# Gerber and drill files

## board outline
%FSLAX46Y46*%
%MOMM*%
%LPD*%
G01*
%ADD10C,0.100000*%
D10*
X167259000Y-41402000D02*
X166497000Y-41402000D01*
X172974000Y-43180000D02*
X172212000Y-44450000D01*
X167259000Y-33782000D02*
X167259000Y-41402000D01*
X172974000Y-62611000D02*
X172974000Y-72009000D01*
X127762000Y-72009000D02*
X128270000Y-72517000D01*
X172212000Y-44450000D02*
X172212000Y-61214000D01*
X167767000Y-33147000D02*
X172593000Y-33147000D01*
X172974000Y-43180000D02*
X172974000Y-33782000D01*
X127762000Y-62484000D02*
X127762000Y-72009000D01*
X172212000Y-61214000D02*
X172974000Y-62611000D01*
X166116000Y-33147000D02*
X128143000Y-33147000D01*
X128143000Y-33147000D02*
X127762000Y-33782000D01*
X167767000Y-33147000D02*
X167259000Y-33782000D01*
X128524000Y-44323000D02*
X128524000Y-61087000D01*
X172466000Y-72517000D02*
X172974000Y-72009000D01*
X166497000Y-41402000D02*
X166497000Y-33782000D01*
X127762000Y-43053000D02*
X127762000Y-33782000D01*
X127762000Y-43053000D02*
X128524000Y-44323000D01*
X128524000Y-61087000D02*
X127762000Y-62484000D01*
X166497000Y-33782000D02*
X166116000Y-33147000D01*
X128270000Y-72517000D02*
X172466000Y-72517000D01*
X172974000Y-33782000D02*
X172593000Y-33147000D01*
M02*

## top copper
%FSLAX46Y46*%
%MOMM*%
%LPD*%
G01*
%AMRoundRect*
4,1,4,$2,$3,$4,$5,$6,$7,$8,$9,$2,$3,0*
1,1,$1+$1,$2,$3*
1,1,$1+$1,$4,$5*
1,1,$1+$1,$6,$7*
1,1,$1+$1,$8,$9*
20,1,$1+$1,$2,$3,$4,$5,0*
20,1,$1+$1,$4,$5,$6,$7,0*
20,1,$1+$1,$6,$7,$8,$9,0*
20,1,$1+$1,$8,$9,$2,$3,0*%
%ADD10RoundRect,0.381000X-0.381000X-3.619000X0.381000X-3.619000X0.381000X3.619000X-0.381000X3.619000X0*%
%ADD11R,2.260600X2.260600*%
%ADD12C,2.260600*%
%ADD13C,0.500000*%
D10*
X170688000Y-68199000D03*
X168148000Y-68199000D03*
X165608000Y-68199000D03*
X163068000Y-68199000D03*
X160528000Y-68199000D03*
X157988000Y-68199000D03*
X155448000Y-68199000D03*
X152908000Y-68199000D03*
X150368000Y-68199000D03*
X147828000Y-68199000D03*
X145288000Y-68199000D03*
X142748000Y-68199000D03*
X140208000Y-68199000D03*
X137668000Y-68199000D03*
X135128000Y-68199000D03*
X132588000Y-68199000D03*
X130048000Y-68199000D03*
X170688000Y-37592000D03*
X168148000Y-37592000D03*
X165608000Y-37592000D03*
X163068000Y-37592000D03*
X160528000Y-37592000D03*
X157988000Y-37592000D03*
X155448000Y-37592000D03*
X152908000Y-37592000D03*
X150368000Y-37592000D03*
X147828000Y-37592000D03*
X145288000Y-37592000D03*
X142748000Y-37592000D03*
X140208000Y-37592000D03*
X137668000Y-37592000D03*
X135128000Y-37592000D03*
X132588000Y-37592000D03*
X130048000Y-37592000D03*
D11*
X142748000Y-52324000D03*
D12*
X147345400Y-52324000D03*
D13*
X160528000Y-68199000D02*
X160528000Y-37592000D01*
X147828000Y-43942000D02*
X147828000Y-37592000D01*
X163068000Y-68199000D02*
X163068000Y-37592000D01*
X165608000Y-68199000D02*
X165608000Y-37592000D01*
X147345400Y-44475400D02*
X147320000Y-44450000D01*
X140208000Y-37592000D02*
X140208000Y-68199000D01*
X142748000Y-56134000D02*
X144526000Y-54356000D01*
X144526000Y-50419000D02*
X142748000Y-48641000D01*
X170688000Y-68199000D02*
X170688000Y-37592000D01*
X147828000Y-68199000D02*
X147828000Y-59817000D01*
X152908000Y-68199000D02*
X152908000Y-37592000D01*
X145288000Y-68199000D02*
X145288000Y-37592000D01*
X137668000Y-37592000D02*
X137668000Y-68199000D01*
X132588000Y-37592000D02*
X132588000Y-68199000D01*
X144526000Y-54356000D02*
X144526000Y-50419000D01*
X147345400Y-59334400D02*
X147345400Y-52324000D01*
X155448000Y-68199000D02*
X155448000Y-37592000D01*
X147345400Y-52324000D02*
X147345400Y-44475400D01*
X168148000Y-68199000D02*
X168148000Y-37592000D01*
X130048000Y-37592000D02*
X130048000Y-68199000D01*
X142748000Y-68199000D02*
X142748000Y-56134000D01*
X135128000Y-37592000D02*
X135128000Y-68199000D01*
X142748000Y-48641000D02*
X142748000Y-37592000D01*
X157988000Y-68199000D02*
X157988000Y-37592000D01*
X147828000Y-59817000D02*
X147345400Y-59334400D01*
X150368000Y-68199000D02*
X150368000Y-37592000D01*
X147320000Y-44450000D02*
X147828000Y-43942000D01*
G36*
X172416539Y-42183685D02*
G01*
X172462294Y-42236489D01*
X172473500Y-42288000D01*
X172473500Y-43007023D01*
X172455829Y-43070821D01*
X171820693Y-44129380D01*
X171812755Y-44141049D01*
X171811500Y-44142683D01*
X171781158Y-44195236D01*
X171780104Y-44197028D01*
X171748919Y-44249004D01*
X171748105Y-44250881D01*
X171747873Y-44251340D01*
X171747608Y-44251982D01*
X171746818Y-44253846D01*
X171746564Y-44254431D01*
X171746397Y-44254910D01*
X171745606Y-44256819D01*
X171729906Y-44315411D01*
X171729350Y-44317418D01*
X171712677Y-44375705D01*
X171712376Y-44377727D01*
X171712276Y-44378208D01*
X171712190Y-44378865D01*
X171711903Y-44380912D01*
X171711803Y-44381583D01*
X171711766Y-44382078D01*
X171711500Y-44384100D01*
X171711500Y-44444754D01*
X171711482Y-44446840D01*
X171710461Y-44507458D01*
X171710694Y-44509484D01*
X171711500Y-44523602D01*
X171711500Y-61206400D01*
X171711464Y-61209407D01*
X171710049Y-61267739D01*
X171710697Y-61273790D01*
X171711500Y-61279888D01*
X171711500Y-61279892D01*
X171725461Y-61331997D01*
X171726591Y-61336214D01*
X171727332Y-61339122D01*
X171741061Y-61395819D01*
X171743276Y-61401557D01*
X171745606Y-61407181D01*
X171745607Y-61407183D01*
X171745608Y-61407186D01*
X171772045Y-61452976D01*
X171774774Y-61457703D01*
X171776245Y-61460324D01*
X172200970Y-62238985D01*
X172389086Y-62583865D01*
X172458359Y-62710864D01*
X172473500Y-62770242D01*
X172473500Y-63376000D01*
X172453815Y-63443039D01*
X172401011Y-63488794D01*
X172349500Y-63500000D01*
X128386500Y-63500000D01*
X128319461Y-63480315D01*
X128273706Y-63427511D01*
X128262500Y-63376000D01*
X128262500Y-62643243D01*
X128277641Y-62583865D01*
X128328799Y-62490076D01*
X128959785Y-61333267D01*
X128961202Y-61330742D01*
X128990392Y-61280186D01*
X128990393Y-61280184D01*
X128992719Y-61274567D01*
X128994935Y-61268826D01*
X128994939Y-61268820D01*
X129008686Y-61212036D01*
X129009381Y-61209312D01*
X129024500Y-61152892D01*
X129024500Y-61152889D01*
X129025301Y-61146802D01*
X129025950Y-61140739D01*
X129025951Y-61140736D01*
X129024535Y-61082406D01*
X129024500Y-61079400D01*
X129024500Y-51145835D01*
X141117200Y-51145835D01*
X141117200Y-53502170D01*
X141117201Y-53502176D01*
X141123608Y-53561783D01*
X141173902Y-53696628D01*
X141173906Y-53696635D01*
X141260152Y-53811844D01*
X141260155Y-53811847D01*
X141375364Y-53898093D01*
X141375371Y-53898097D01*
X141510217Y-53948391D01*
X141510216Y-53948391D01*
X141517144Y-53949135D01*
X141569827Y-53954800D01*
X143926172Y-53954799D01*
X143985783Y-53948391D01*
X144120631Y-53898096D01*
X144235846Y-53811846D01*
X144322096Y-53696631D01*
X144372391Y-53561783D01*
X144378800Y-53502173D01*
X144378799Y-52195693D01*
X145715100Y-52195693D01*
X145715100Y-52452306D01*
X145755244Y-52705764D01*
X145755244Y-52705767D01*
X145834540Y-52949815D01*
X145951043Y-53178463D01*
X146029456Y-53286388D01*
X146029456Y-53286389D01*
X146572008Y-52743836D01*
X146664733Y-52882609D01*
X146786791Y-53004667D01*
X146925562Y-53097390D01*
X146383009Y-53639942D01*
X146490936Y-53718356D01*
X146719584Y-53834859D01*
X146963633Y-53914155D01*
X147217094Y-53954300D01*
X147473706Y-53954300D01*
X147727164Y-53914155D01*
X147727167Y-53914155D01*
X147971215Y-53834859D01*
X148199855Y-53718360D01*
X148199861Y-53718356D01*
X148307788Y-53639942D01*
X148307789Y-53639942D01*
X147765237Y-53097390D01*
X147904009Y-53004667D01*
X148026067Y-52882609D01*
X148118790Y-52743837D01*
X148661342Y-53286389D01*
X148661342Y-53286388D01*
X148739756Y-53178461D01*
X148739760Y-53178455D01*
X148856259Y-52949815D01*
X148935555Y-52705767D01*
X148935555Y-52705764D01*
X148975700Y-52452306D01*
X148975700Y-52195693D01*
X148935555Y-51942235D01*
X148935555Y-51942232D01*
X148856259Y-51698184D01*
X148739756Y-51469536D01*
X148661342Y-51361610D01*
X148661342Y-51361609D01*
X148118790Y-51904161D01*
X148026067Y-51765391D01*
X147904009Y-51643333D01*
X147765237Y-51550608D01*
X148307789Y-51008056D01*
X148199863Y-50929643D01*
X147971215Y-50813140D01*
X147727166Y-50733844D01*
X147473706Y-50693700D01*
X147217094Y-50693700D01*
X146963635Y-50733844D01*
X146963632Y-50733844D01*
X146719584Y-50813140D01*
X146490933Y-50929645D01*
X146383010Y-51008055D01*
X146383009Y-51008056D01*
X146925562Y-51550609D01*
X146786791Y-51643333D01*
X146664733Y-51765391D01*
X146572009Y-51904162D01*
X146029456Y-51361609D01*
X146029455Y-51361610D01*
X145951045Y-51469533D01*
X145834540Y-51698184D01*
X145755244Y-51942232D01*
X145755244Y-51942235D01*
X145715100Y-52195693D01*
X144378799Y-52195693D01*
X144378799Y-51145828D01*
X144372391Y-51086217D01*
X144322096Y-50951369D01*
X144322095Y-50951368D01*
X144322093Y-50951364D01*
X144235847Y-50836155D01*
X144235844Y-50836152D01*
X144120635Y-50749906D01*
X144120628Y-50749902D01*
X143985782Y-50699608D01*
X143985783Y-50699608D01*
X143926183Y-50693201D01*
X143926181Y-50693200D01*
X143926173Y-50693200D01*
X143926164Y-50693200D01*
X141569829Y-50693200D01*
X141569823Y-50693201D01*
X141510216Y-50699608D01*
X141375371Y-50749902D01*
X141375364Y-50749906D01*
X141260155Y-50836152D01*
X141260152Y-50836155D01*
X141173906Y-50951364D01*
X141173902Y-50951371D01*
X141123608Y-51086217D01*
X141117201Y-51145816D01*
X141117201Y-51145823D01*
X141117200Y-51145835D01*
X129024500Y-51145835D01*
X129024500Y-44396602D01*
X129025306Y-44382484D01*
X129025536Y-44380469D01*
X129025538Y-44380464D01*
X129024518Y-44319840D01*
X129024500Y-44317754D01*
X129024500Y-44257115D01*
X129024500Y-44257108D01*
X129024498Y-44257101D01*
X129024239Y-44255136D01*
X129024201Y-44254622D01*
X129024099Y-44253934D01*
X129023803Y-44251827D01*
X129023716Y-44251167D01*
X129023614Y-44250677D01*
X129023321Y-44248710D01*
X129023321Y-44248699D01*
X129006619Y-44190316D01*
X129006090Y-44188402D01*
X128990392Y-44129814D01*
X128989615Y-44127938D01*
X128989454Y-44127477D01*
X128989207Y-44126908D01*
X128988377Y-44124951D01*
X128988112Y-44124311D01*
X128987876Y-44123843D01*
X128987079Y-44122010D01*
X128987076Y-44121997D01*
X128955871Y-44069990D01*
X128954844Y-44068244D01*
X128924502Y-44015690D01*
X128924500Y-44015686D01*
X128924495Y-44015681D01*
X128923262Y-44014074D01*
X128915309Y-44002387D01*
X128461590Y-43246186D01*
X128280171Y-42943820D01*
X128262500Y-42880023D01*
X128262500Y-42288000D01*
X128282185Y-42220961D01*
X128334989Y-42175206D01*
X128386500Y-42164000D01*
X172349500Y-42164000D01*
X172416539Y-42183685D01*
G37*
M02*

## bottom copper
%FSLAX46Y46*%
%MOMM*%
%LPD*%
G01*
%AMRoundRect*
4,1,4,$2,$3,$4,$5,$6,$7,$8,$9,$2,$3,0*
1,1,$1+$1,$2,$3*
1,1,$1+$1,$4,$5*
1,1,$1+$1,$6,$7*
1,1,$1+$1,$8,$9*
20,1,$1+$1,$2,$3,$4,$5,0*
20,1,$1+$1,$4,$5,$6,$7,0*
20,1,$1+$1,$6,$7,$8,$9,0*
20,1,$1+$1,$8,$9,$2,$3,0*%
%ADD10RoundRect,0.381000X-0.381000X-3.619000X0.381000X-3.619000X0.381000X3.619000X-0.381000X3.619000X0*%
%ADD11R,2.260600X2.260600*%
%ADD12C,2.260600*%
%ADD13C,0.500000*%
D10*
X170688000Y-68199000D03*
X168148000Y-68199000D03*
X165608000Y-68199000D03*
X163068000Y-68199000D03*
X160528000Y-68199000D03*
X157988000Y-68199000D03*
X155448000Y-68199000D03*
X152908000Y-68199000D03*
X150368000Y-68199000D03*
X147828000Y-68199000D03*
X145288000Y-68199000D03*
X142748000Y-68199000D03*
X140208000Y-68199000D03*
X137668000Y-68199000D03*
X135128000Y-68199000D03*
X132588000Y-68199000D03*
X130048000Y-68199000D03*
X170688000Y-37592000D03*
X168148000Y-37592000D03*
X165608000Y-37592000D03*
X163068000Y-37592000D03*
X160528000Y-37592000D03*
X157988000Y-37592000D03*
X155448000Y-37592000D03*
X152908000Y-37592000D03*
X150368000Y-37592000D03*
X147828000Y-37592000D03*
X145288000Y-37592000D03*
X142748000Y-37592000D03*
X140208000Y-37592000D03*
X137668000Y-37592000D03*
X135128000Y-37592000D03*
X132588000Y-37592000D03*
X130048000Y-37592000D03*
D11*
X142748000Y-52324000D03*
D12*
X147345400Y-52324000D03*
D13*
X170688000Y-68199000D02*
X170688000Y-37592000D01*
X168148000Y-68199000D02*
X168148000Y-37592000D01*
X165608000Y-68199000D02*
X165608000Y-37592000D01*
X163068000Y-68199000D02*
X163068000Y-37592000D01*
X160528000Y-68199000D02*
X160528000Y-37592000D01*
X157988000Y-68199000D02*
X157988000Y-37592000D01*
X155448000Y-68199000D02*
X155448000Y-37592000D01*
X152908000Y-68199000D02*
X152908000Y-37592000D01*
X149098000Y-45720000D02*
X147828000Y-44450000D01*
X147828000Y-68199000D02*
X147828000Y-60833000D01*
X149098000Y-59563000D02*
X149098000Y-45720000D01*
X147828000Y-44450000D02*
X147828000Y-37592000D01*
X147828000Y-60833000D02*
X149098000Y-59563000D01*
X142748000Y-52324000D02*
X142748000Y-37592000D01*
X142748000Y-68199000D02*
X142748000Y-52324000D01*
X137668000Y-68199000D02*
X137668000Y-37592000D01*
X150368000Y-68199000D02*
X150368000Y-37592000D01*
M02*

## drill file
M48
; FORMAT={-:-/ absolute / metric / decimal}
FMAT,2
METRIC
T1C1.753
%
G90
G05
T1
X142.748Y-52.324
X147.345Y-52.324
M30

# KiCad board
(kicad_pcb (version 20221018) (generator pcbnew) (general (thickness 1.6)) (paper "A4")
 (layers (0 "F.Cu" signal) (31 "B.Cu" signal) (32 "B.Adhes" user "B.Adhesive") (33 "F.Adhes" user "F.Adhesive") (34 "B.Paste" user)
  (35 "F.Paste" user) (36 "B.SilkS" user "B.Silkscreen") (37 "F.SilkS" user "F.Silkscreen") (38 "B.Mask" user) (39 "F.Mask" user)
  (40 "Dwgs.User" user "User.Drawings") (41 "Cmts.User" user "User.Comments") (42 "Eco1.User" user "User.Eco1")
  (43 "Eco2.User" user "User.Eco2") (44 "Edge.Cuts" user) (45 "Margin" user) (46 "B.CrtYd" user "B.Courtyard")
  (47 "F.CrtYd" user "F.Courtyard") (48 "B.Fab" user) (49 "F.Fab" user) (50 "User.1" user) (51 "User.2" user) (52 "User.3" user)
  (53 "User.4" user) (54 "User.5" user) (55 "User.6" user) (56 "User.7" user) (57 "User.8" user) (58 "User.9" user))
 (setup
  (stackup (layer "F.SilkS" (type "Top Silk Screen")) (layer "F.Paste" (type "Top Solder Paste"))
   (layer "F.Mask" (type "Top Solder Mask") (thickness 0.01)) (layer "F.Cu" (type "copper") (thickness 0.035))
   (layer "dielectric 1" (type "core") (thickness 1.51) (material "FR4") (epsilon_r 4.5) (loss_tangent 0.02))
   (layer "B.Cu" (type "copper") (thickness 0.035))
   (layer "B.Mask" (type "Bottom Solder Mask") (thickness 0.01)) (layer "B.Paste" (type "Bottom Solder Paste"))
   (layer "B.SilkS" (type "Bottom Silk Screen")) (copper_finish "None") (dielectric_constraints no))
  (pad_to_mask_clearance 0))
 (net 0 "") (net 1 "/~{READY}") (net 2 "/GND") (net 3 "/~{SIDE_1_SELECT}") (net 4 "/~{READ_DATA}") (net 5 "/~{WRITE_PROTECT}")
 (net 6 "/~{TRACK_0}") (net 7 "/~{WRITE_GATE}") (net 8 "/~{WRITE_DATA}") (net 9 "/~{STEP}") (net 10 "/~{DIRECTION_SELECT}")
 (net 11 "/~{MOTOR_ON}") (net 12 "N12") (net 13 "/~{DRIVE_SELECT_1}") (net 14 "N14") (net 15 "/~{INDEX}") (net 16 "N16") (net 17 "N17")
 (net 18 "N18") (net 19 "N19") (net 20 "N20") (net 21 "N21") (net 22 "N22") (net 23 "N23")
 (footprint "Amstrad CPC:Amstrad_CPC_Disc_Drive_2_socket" (layer "F.Cu") (at 157.988 74.803)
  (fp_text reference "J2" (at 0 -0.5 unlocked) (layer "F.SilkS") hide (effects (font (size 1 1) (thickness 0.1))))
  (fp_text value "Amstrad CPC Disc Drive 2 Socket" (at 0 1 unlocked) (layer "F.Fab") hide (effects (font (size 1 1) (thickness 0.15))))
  (pad "1" smd roundrect (at 12.7 -6.604) (size 1.524 8) (layers "B.Cu" "B.Paste" "B.Mask") (roundrect_rratio 0.25) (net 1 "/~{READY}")
   (thermal_bridge_angle 45))
  (pad "2" smd roundrect (at 12.7 -6.604) (size 1.524 8) (layers "F.Cu" "F.Paste" "F.Mask") (roundrect_rratio 0.25) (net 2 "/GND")
   (thermal_bridge_angle 45))
  (pad "3" smd roundrect (at 10.16 -6.604) (size 1.524 8) (layers "B.Cu" "B.Paste" "B.Mask") (roundrect_rratio 0.25)
   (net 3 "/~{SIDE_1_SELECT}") (thermal_bridge_angle 45))
  (pad "4" smd roundrect (at 10.16 -6.604) (size 1.524 8) (layers "F.Cu" "F.Paste" "F.Mask") (roundrect_rratio 0.25) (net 2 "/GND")
   (thermal_bridge_angle 45))
  (pad "5" smd roundrect (at 7.62 -6.604) (size 1.524 8) (layers "B.Cu" "B.Paste" "B.Mask") (roundrect_rratio 0.25) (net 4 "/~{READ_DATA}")
   (thermal_bridge_angle 45))
  (pad "6" smd roundrect (at 7.62 -6.604) (size 1.524 8) (layers "F.Cu" "F.Paste" "F.Mask") (roundrect_rratio 0.25) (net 2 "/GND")
   (thermal_bridge_angle 45))
  (pad "7" smd roundrect (at 5.08 -6.604) (size 1.524 8) (layers "B.Cu" "B.Paste" "B.Mask") (roundrect_rratio 0.25)
   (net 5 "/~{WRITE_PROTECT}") (thermal_bridge_angle 45))
  (pad "8" smd roundrect (at 5.08 -6.604) (size 1.524 8) (layers "F.Cu" "F.Paste" "F.Mask") (roundrect_rratio 0.25) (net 2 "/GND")
   (thermal_bridge_angle 45))
  (pad "9" smd roundrect (at 2.54 -6.604) (size 1.524 8) (layers "B.Cu" "B.Paste" "B.Mask") (roundrect_rratio 0.25) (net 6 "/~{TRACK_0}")
   (thermal_bridge_angle 45))
  (pad "10" smd roundrect (at 2.54 -6.604) (size 1.524 8) (layers "F.Cu" "F.Paste" "F.Mask") (roundrect_rratio 0.25) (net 2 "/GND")
   (thermal_bridge_angle 45))
  (pad "11" smd roundrect (at 0 -6.604) (size 1.524 8) (layers "B.Cu" "B.Paste" "B.Mask") (roundrect_rratio 0.25) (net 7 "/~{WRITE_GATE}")
   (thermal_bridge_angle 45))
  (pad "12" smd roundrect (at 0 -6.604) (size 1.524 8) (layers "F.Cu" "F.Paste" "F.Mask") (roundrect_rratio 0.25) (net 2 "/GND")
   (thermal_bridge_angle 45))
  (pad "13" smd roundrect (at -2.54 -6.604) (size 1.524 8) (layers "B.Cu" "B.Paste" "B.Mask") (roundrect_rratio 0.25)
   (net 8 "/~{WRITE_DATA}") (thermal_bridge_angle 45))
  (pad "14" smd roundrect (at -2.54 -6.604) (size 1.524 8) (layers "F.Cu" "F.Paste" "F.Mask") (roundrect_rratio 0.25) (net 2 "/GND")
   (thermal_bridge_angle 45))
  (pad "15" smd roundrect (at -5.08 -6.604) (size 1.524 8) (layers "B.Cu" "B.Paste" "B.Mask") (roundrect_rratio 0.25) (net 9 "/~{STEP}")
   (thermal_bridge_angle 45))
  (pad "16" smd roundrect (at -5.08 -6.604) (size 1.524 8) (layers "F.Cu" "F.Paste" "F.Mask") (roundrect_rratio 0.25) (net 2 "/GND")
   (thermal_bridge_angle 45))
  (pad "17" smd roundrect (at -7.62 -6.604) (size 1.524 8) (layers "B.Cu" "B.Paste" "B.Mask") (roundrect_rratio 0.25)
   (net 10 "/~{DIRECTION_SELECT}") (thermal_bridge_angle 45))
  (pad "18" smd roundrect (at -7.62 -6.604) (size 1.524 8) (layers "F.Cu" "F.Paste" "F.Mask") (roundrect_rratio 0.25) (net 2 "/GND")
   (thermal_bridge_angle 45))
  (pad "19" smd roundrect (at -10.16 -6.604) (size 1.524 8) (layers "B.Cu" "B.Paste" "B.Mask") (roundrect_rratio 0.25)
   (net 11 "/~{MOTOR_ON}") (thermal_bridge_angle 45))
  (pad "20" smd roundrect (at -10.16 -6.604) (size 1.524 8) (layers "F.Cu" "F.Paste" "F.Mask") (roundrect_rratio 0.25) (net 2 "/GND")
   (thermal_bridge_angle 45))
  (pad "21" smd roundrect (at -12.7 -6.604) (size 1.524 8) (layers "B.Cu" "B.Paste" "B.Mask") (roundrect_rratio 0.25) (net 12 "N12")
   (thermal_bridge_angle 45))
  (pad "22" smd roundrect (at -12.7 -6.604) (size 1.524 8) (layers "F.Cu" "F.Paste" "F.Mask") (roundrect_rratio 0.25) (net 2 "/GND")
   (thermal_bridge_angle 45))
  (pad "23" smd roundrect (at -15.24 -6.604) (size 1.524 8) (layers "B.Cu" "B.Paste" "B.Mask") (roundrect_rratio 0.25)
   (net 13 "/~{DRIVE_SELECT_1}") (thermal_bridge_angle 45))
  (pad "24" smd roundrect (at -15.24 -6.604) (size 1.524 8) (layers "F.Cu" "F.Paste" "F.Mask") (roundrect_rratio 0.25) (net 2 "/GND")
   (thermal_bridge_angle 45))
  (pad "25" smd roundrect (at -17.78 -6.604) (size 1.524 8) (layers "B.Cu" "B.Paste" "B.Mask") (roundrect_rratio 0.25) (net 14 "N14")
   (thermal_bridge_angle 45))
  (pad "26" smd roundrect (at -17.78 -6.604) (size 1.524 8) (layers "F.Cu" "F.Paste" "F.Mask") (roundrect_rratio 0.25) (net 2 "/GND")
   (thermal_bridge_angle 45))
  (pad "27" smd roundrect (at -20.32 -6.604) (size 1.524 8) (layers "B.Cu" "B.Paste" "B.Mask") (roundrect_rratio 0.25) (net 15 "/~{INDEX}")
   (thermal_bridge_angle 45))
  (pad "28" smd roundrect (at -20.32 -6.604) (size 1.524 8) (layers "F.Cu" "F.Paste" "F.Mask") (roundrect_rratio 0.25) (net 2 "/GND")
   (thermal_bridge_angle 45))
  (pad "29" smd roundrect (at -22.86 -6.604) (size 1.524 8) (layers "B.Cu" "B.Paste" "B.Mask") (roundrect_rratio 0.25) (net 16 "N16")
   (thermal_bridge_angle 45))
  (pad "30" smd roundrect (at -22.86 -6.604) (size 1.524 8) (layers "F.Cu" "F.Paste" "F.Mask") (roundrect_rratio 0.25) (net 2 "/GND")
   (thermal_bridge_angle 45))
  (pad "31" smd roundrect (at -25.4 -6.604) (size 1.524 8) (layers "B.Cu" "B.Paste" "B.Mask") (roundrect_rratio 0.25) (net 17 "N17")
   (thermal_bridge_angle 45))
  (pad "32" smd roundrect (at -25.4 -6.604) (size 1.524 8) (layers "F.Cu" "F.Paste" "F.Mask") (roundrect_rratio 0.25) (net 2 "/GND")
   (thermal_bridge_angle 45))
  (pad "33" smd roundrect (at -27.94 -6.604) (size 1.524 8) (layers "B.Cu" "B.Paste" "B.Mask") (roundrect_rratio 0.25) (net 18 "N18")
   (thermal_bridge_angle 45))
  (pad "34" smd roundrect (at -27.94 -6.604) (size 1.524 8) (layers "F.Cu" "F.Paste" "F.Mask") (roundrect_rratio 0.25) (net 2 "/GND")
   (thermal_bridge_angle 45)))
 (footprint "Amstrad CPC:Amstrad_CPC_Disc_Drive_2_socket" (layer "F.Cu") (at 157.988 44.196)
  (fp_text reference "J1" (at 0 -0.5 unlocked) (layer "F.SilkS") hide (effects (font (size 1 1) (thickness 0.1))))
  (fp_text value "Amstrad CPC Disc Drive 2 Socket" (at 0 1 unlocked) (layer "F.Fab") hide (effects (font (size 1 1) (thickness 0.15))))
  (pad "1" smd roundrect (at 12.7 -6.604) (size 1.524 8) (layers "B.Cu" "B.Paste" "B.Mask") (roundrect_rratio 0.25) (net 1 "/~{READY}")
   (thermal_bridge_angle 45))
  (pad "2" smd roundrect (at 12.7 -6.604) (size 1.524 8) (layers "F.Cu" "F.Paste" "F.Mask") (roundrect_rratio 0.25) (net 2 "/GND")
   (thermal_bridge_angle 45))
  (pad "3" smd roundrect (at 10.16 -6.604) (size 1.524 8) (layers "B.Cu" "B.Paste" "B.Mask") (roundrect_rratio 0.25)
   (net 3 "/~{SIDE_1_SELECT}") (thermal_bridge_angle 45))
  (pad "4" smd roundrect (at 10.16 -6.604) (size 1.524 8) (layers "F.Cu" "F.Paste" "F.Mask") (roundrect_rratio 0.25) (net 2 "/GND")
   (thermal_bridge_angle 45))
  (pad "5" smd roundrect (at 7.62 -6.604) (size 1.524 8) (layers "B.Cu" "B.Paste" "B.Mask") (roundrect_rratio 0.25) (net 4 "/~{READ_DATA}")
   (thermal_bridge_angle 45))
  (pad "6" smd roundrect (at 7.62 -6.604) (size 1.524 8) (layers "F.Cu" "F.Paste" "F.Mask") (roundrect_rratio 0.25) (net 2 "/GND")
   (thermal_bridge_angle 45))
  (pad "7" smd roundrect (at 5.08 -6.604) (size 1.524 8) (layers "B.Cu" "B.Paste" "B.Mask") (roundrect_rratio 0.25)
   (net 5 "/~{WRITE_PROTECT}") (thermal_bridge_angle 45))
  (pad "8" smd roundrect (at 5.08 -6.604) (size 1.524 8) (layers "F.Cu" "F.Paste" "F.Mask") (roundrect_rratio 0.25) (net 2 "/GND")
   (thermal_bridge_angle 45))
  (pad "9" smd roundrect (at 2.54 -6.604) (size 1.524 8) (layers "B.Cu" "B.Paste" "B.Mask") (roundrect_rratio 0.25) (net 6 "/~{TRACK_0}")
   (thermal_bridge_angle 45))
  (pad "10" smd roundrect (at 2.54 -6.604) (size 1.524 8) (layers "F.Cu" "F.Paste" "F.Mask") (roundrect_rratio 0.25) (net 2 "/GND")
   (thermal_bridge_angle 45))
  (pad "11" smd roundrect (at 0 -6.604) (size 1.524 8) (layers "B.Cu" "B.Paste" "B.Mask") (roundrect_rratio 0.25) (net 7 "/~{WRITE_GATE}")
   (thermal_bridge_angle 45))
  (pad "12" smd roundrect (at 0 -6.604) (size 1.524 8) (layers "F.Cu" "F.Paste" "F.Mask") (roundrect_rratio 0.25) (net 2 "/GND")
   (thermal_bridge_angle 45))
  (pad "13" smd roundrect (at -2.54 -6.604) (size 1.524 8) (layers "B.Cu" "B.Paste" "B.Mask") (roundrect_rratio 0.25)
   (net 8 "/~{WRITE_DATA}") (thermal_bridge_angle 45))
  (pad "14" smd roundrect (at -2.54 -6.604) (size 1.524 8) (layers "F.Cu" "F.Paste" "F.Mask") (roundrect_rratio 0.25) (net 2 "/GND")
   (thermal_bridge_angle 45))
  (pad "15" smd roundrect (at -5.08 -6.604) (size 1.524 8) (layers "B.Cu" "B.Paste" "B.Mask") (roundrect_rratio 0.25) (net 9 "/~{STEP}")
   (thermal_bridge_angle 45))
  (pad "16" smd roundrect (at -5.08 -6.604) (size 1.524 8) (layers "F.Cu" "F.Paste" "F.Mask") (roundrect_rratio 0.25) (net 2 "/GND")
   (thermal_bridge_angle 45))
  (pad "17" smd roundrect (at -7.62 -6.604) (size 1.524 8) (layers "B.Cu" "B.Paste" "B.Mask") (roundrect_rratio 0.25)
   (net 10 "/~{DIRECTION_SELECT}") (thermal_bridge_angle 45))
  (pad "18" smd roundrect (at -7.62 -6.604) (size 1.524 8) (layers "F.Cu" "F.Paste" "F.Mask") (roundrect_rratio 0.25) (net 2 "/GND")
   (thermal_bridge_angle 45))
  (pad "19" smd roundrect (at -10.16 -6.604) (size 1.524 8) (layers "B.Cu" "B.Paste" "B.Mask") (roundrect_rratio 0.25)
   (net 11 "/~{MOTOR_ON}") (thermal_bridge_angle 45))
  (pad "20" smd roundrect (at -10.16 -6.604) (size 1.524 8) (layers "F.Cu" "F.Paste" "F.Mask") (roundrect_rratio 0.25) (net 2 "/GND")
   (thermal_bridge_angle 45))
  (pad "21" smd roundrect (at -12.7 -6.604) (size 1.524 8) (layers "B.Cu" "B.Paste" "B.Mask") (roundrect_rratio 0.25) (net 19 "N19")
   (thermal_bridge_angle 45))
  (pad "22" smd roundrect (at -12.7 -6.604) (size 1.524 8) (layers "F.Cu" "F.Paste" "F.Mask") (roundrect_rratio 0.25) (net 2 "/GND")
   (thermal_bridge_angle 45))
  (pad "23" smd roundrect (at -15.24 -6.604) (size 1.524 8) (layers "B.Cu" "B.Paste" "B.Mask") (roundrect_rratio 0.25)
   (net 13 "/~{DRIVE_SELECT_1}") (thermal_bridge_angle 45))
  (pad "24" smd roundrect (at -15.24 -6.604) (size 1.524 8) (layers "F.Cu" "F.Paste" "F.Mask") (roundrect_rratio 0.25) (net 2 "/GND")
   (thermal_bridge_angle 45))
  (pad "25" smd roundrect (at -17.78 -6.604) (size 1.524 8) (layers "B.Cu" "B.Paste" "B.Mask") (roundrect_rratio 0.25) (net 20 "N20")
   (thermal_bridge_angle 45))
  (pad "26" smd roundrect (at -17.78 -6.604) (size 1.524 8) (layers "F.Cu" "F.Paste" "F.Mask") (roundrect_rratio 0.25) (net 2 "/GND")
   (thermal_bridge_angle 45))
  (pad "27" smd roundrect (at -20.32 -6.604) (size 1.524 8) (layers "B.Cu" "B.Paste" "B.Mask") (roundrect_rratio 0.25) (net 15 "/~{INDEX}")
   (thermal_bridge_angle 45))
  (pad "28" smd roundrect (at -20.32 -6.604) (size 1.524 8) (layers "F.Cu" "F.Paste" "F.Mask") (roundrect_rratio 0.25) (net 2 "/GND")
   (thermal_bridge_angle 45))
  (pad "29" smd roundrect (at -22.86 -6.604) (size 1.524 8) (layers "B.Cu" "B.Paste" "B.Mask") (roundrect_rratio 0.25) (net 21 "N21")
   (thermal_bridge_angle 45))
  (pad "30" smd roundrect (at -22.86 -6.604) (size 1.524 8) (layers "F.Cu" "F.Paste" "F.Mask") (roundrect_rratio 0.25) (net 2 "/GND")
   (thermal_bridge_angle 45))
  (pad "31" smd roundrect (at -25.4 -6.604) (size 1.524 8) (layers "B.Cu" "B.Paste" "B.Mask") (roundrect_rratio 0.25) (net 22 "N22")
   (thermal_bridge_angle 45))
  (pad "32" smd roundrect (at -25.4 -6.604) (size 1.524 8) (layers "F.Cu" "F.Paste" "F.Mask") (roundrect_rratio 0.25) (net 2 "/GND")
   (thermal_bridge_angle 45))
  (pad "33" smd roundrect (at -27.94 -6.604) (size 1.524 8) (layers "B.Cu" "B.Paste" "B.Mask") (roundrect_rratio 0.25) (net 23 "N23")
   (thermal_bridge_angle 45))
  (pad "34" smd roundrect (at -27.94 -6.604) (size 1.524 8) (layers "F.Cu" "F.Paste" "F.Mask") (roundrect_rratio 0.25) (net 2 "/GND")
   (thermal_bridge_angle 45)))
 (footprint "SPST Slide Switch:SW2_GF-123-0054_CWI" (layer "F.Cu") (at 142.748 52.324 90)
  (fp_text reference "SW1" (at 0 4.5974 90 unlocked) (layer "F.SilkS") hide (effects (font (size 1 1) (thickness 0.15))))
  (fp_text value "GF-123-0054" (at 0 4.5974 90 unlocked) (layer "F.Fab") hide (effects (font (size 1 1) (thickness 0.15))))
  (pad "1" thru_hole rect (at 0 0 90) (size 2.2606 2.2606) (drill 1.7526) (layers "*.Cu" "*.Mask") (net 13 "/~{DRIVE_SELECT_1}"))
  (pad "2" thru_hole circle (at 0 4.5974 90) (size 2.2606 2.2606) (drill 1.7526) (layers "*.Cu" "*.Mask") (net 2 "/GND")))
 (gr_line (start 167.259 41.402) (end 166.497 41.402) (stroke (width 0.1) (type default)) (layer "Edge.Cuts"))
 (gr_line (start 172.974 43.18) (end 172.212 44.45) (stroke (width 0.1) (type default)) (layer "Edge.Cuts"))
 (gr_line (start 167.259 33.782) (end 167.259 41.402) (stroke (width 0.1) (type default)) (layer "Edge.Cuts"))
 (gr_line (start 172.974 62.611) (end 172.974 72.009) (stroke (width 0.1) (type default)) (layer "Edge.Cuts"))
 (gr_line (start 127.762 72.009) (end 128.27 72.517) (stroke (width 0.1) (type default)) (layer "Edge.Cuts"))
 (gr_line (start 172.212 44.45) (end 172.212 61.214) (stroke (width 0.1) (type default)) (layer "Edge.Cuts"))
 (gr_line (start 167.767 33.147) (end 172.593 33.147) (stroke (width 0.1) (type default)) (layer "Edge.Cuts"))
 (gr_line (start 172.974 43.18) (end 172.974 33.782) (stroke (width 0.1) (type default)) (layer "Edge.Cuts"))
 (gr_line (start 127.762 62.484) (end 127.762 72.009) (stroke (width 0.1) (type default)) (layer "Edge.Cuts"))
 (gr_line (start 172.212 61.214) (end 172.974 62.611) (stroke (width 0.1) (type default)) (layer "Edge.Cuts"))
 (gr_line (start 166.116 33.147) (end 128.143 33.147) (stroke (width 0.1) (type default)) (layer "Edge.Cuts"))
 (gr_line (start 128.143 33.147) (end 127.762 33.782) (stroke (width 0.1) (type default)) (layer "Edge.Cuts"))
 (gr_line (start 167.767 33.147) (end 167.259 33.782) (stroke (width 0.1) (type default)) (layer "Edge.Cuts"))
 (gr_line (start 128.524 44.323) (end 128.524 61.087) (stroke (width 0.1) (type default)) (layer "Edge.Cuts"))
 (gr_line (start 172.466 72.517) (end 172.974 72.009) (stroke (width 0.1) (type default)) (layer "Edge.Cuts"))
 (gr_line (start 166.497 41.402) (end 166.497 33.782) (stroke (width 0.1) (type default)) (layer "Edge.Cuts"))
 (gr_line (start 127.762 43.053) (end 127.762 33.782) (stroke (width 0.1) (type default)) (layer "Edge.Cuts"))
 (gr_line (start 127.762 43.053) (end 128.524 44.323) (stroke (width 0.1) (type default)) (layer "Edge.Cuts"))
 (gr_line (start 128.524 61.087) (end 127.762 62.484) (stroke (width 0.1) (type default)) (layer "Edge.Cuts"))
 (gr_line (start 166.497 33.782) (end 166.116 33.147) (stroke (width 0.1) (type default)) (layer "Edge.Cuts"))
 (gr_line (start 128.27 72.517) (end 172.466 72.517) (stroke (width 0.1) (type default)) (layer "Edge.Cuts"))
 (gr_line (start 172.974 33.782) (end 172.593 33.147) (stroke (width 0.1) (type default)) (layer "Edge.Cuts"))
 (segment (start 170.688 68.199) (end 170.688 37.592) (width 0.5) (layer "B.Cu") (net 1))
 (segment (start 160.528 68.199) (end 160.528 37.592) (width 0.5) (layer "F.Cu") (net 2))
 (segment (start 147.828 43.942) (end 147.828 37.592) (width 0.5) (layer "F.Cu") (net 2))
 (segment (start 163.068 68.199) (end 163.068 37.592) (width 0.5) (layer "F.Cu") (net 2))
 (segment (start 165.608 68.199) (end 165.608 37.592) (width 0.5) (layer "F.Cu") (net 2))
 (segment (start 147.3454 44.4754) (end 147.32 44.45) (width 0.5) (layer "F.Cu") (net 2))
 (segment (start 140.208 37.592) (end 140.208 68.199) (width 0.5) (layer "F.Cu") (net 2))
 (segment (start 142.748 56.134) (end 144.526 54.356) (width 0.5) (layer "F.Cu") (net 2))
 (segment (start 144.526 50.419) (end 142.748 48.641) (width 0.5) (layer "F.Cu") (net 2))
 (segment (start 170.688 68.199) (end 170.688 37.592) (width 0.5) (layer "F.Cu") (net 2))
 (segment (start 147.828 68.199) (end 147.828 59.817) (width 0.5) (layer "F.Cu") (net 2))
 (segment (start 152.908 68.199) (end 152.908 37.592) (width 0.5) (layer "F.Cu") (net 2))
 (segment (start 145.288 68.199) (end 145.288 37.592) (width 0.5) (layer "F.Cu") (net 2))
 (segment (start 137.668 37.592) (end 137.668 68.199) (width 0.5) (layer "F.Cu") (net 2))
 (segment (start 132.588 37.592) (end 132.588 68.199) (width 0.5) (layer "F.Cu") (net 2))
 (segment (start 144.526 54.356) (end 144.526 50.419) (width 0.5) (layer "F.Cu") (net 2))
 (segment (start 147.3454 59.3344) (end 147.3454 52.324) (width 0.5) (layer "F.Cu") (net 2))
 (segment (start 155.448 68.199) (end 155.448 37.592) (width 0.5) (layer "F.Cu") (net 2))
 (segment (start 147.3454 52.324) (end 147.3454 44.4754) (width 0.5) (layer "F.Cu") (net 2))
 (segment (start 168.148 68.199) (end 168.148 37.592) (width 0.5) (layer "F.Cu") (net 2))
 (segment (start 130.048 37.592) (end 130.048 68.199) (width 0.5) (layer "F.Cu") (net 2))
 (segment (start 142.748 68.199) (end 142.748 56.134) (width 0.5) (layer "F.Cu") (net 2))
 (segment (start 135.128 37.592) (end 135.128 68.199) (width 0.5) (layer "F.Cu") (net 2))
 (segment (start 142.748 48.641) (end 142.748 37.592) (width 0.5) (layer "F.Cu") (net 2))
 (segment (start 157.988 68.199) (end 157.988 37.592) (width 0.5) (layer "F.Cu") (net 2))
 (segment (start 147.828 59.817) (end 147.3454 59.3344) (width 0.5) (layer "F.Cu") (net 2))
 (segment (start 150.368 68.199) (end 150.368 37.592) (width 0.5) (layer "F.Cu") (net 2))
 (segment (start 147.32 44.45) (end 147.828 43.942) (width 0.5) (layer "F.Cu") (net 2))
 (segment (start 168.148 68.199) (end 168.148 37.592) (width 0.5) (layer "B.Cu") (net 3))
 (segment (start 165.608 68.199) (end 165.608 37.592) (width 0.5) (layer "B.Cu") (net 4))
 (segment (start 163.068 68.199) (end 163.068 37.592) (width 0.5) (layer "B.Cu") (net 5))
 (segment (start 160.528 68.199) (end 160.528 37.592) (width 0.5) (layer "B.Cu") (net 6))
 (segment (start 157.988 68.199) (end 157.988 37.592) (width 0.5) (layer "B.Cu") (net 7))
 (segment (start 155.448 68.199) (end 155.448 37.592) (width 0.5) (layer "B.Cu") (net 8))
 (segment (start 152.908 68.199) (end 152.908 37.592) (width 0.5) (layer "B.Cu") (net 9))
 (segment (start 149.098 45.72) (end 147.828 44.45) (width 0.5) (layer "B.Cu") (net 11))
 (segment (start 147.828 68.199) (end 147.828 60.833) (width 0.5) (layer "B.Cu") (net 11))
 (segment (start 149.098 59.563) (end 149.098 45.72) (width 0.5) (layer "B.Cu") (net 11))
 (segment (start 147.828 44.45) (end 147.828 37.592) (width 0.5) (layer "B.Cu") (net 11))
 (segment (start 147.828 60.833) (end 149.098 59.563) (width 0.5) (layer "B.Cu") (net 11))
 (segment (start 142.748 52.324) (end 142.748 37.592) (width 0.5) (layer "B.Cu") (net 13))
 (segment (start 142.748 68.199) (end 142.748 52.324) (width 0.5) (layer "B.Cu") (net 13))
 (segment (start 137.668 68.199) (end 137.668 37.592) (width 0.5) (layer "B.Cu") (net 15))
 (segment (start 150.368 68.199) (end 150.368 37.592) (width 0.5) (layer "B.Cu") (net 10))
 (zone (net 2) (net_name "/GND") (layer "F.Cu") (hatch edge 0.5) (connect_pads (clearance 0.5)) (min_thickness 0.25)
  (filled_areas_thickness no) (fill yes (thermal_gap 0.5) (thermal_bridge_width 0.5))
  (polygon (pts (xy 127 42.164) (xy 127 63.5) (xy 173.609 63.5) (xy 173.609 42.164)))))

